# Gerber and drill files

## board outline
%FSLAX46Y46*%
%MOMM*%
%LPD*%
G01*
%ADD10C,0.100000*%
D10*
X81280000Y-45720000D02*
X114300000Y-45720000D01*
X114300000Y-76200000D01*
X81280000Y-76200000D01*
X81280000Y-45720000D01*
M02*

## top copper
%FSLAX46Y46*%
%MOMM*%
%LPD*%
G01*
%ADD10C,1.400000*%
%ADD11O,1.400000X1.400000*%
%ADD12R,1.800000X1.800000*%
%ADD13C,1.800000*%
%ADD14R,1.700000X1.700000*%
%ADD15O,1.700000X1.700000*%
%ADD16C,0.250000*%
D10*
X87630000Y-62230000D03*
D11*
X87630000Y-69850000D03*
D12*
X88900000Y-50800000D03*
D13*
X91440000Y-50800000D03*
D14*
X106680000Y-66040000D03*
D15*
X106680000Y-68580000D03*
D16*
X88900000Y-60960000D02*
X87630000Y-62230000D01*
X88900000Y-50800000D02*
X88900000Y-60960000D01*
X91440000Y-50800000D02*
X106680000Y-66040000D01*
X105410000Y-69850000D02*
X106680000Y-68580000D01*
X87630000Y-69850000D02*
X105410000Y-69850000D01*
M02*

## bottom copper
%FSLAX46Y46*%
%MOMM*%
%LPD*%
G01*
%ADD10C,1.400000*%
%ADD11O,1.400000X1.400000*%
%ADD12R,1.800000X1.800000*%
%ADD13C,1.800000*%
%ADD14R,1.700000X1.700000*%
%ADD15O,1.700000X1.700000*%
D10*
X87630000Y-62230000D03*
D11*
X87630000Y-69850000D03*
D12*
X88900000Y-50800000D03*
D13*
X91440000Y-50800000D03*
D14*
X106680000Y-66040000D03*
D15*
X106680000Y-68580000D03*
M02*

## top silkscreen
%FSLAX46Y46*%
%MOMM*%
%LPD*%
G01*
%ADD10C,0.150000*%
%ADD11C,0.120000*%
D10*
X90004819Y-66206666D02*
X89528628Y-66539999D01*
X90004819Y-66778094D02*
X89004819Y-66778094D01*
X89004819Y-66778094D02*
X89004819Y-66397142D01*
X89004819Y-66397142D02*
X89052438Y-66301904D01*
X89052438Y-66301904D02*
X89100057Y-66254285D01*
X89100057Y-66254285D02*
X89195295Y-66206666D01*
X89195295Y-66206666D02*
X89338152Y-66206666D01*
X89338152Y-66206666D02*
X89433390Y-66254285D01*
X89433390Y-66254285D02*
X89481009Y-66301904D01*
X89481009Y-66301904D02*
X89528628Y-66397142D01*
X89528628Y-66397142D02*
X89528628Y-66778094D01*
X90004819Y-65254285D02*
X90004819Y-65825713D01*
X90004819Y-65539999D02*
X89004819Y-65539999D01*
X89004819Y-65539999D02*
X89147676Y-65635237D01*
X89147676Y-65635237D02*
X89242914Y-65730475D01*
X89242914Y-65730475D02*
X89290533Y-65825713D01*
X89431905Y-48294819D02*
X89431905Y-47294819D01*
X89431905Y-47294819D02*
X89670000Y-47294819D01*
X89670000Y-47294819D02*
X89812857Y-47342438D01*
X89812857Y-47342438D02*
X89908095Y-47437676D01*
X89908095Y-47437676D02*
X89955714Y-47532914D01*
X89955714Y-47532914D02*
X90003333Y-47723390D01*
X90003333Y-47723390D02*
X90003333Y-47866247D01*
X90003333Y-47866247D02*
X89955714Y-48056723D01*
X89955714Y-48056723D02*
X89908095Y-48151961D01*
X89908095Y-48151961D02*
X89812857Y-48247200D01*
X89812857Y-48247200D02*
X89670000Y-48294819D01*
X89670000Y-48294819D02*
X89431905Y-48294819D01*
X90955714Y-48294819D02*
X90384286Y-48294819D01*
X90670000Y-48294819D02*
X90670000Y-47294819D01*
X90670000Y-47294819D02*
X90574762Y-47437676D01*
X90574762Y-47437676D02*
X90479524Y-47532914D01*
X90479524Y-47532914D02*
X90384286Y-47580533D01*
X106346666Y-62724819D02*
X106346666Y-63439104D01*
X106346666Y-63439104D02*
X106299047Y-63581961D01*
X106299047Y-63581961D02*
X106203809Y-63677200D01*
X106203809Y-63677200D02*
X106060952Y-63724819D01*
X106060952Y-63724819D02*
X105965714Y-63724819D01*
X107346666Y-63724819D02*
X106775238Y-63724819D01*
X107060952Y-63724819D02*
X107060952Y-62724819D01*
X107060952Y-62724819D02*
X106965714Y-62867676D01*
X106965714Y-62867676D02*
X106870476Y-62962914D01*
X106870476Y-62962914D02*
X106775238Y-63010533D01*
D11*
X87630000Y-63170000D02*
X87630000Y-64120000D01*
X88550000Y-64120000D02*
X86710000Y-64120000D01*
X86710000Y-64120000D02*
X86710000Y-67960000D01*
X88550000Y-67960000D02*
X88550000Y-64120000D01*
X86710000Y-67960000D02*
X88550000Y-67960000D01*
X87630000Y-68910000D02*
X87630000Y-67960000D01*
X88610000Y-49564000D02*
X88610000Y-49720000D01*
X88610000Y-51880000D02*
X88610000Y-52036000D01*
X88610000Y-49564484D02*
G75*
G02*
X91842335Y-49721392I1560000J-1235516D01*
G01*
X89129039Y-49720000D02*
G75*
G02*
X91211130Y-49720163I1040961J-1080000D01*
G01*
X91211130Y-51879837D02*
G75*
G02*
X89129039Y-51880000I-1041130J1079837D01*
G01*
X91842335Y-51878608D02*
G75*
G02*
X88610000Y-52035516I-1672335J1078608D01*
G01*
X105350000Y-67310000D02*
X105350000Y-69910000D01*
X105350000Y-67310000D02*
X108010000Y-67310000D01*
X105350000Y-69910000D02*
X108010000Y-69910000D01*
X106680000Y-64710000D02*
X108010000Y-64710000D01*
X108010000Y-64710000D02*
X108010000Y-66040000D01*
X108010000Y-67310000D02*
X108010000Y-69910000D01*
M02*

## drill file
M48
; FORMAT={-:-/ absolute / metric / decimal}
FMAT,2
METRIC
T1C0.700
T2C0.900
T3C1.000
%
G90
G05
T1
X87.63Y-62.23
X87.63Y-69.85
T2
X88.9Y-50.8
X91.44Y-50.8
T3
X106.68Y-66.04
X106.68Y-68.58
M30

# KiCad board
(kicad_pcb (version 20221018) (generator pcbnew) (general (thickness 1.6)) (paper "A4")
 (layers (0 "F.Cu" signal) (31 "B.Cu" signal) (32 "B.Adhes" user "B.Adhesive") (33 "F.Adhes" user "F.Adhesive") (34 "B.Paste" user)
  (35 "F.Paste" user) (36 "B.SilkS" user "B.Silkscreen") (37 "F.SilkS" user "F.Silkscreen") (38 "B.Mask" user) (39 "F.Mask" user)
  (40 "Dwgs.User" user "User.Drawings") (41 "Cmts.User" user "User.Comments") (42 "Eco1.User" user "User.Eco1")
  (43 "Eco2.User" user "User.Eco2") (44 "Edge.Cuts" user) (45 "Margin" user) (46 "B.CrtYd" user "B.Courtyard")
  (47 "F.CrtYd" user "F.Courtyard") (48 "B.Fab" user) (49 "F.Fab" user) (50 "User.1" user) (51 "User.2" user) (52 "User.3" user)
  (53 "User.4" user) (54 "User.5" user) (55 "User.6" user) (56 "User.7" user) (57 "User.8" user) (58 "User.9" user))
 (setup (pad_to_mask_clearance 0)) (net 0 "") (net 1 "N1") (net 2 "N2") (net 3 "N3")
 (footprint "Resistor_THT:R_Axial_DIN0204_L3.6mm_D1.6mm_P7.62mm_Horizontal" (layer "F.Cu") (at 87.63 62.23 -90)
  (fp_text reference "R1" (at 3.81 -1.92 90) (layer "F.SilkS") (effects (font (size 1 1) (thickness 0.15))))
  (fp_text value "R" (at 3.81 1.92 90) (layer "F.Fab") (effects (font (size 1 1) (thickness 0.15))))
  (fp_line (start 0.94 0) (end 1.89 0) (stroke (width 0.12) (type solid)) (layer "F.SilkS"))
  (fp_line (start 1.89 -0.92) (end 1.89 0.92) (stroke (width 0.12) (type solid)) (layer "F.SilkS"))
  (fp_line (start 1.89 0.92) (end 5.73 0.92) (stroke (width 0.12) (type solid)) (layer "F.SilkS"))
  (fp_line (start 5.73 -0.92) (end 1.89 -0.92) (stroke (width 0.12) (type solid)) (layer "F.SilkS"))
  (fp_line (start 5.73 0.92) (end 5.73 -0.92) (stroke (width 0.12) (type solid)) (layer "F.SilkS"))
  (fp_line (start 6.68 0) (end 5.73 0) (stroke (width 0.12) (type solid)) (layer "F.SilkS"))
  (pad "1" thru_hole circle (at 0 0 270) (size 1.4 1.4) (drill 0.7) (layers "*.Cu" "*.Mask") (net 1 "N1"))
  (pad "2" thru_hole oval (at 7.62 0 270) (size 1.4 1.4) (drill 0.7) (layers "*.Cu" "*.Mask") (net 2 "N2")))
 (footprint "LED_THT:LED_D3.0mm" (layer "F.Cu") (at 88.9 50.8)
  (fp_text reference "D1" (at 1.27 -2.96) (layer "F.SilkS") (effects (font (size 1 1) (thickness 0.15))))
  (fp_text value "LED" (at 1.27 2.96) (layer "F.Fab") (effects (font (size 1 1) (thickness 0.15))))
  (fp_line (start -0.29 -1.236) (end -0.29 -1.08) (stroke (width 0.12) (type solid)) (layer "F.SilkS"))
  (fp_line (start -0.29 1.08) (end -0.29 1.236) (stroke (width 0.12) (type solid)) (layer "F.SilkS"))
  (fp_arc (start -0.29 -1.235516) (mid 1.366487 -1.987659) (end 2.942335 -1.078608) (stroke (width 0.12) (type solid)) (layer "F.SilkS"))
  (fp_arc (start 0.229039 -1.08) (mid 1.270117 -1.5) (end 2.31113 -1.079837) (stroke (width 0.12) (type solid)) (layer "F.SilkS"))
  (fp_arc (start 2.31113 1.079837) (mid 1.270117 1.5) (end 0.229039 1.08) (stroke (width 0.12) (type solid)) (layer "F.SilkS"))
  (fp_arc (start 2.942335 1.078608) (mid 1.366487 1.987659) (end -0.29 1.235516) (stroke (width 0.12) (type solid)) (layer "F.SilkS"))
  (pad "1" thru_hole rect (at 0 0) (size 1.8 1.8) (drill 0.9) (layers "*.Cu" "*.Mask") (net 1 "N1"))
  (pad "2" thru_hole circle (at 2.54 0) (size 1.8 1.8) (drill 0.9) (layers "*.Cu" "*.Mask") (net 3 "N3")))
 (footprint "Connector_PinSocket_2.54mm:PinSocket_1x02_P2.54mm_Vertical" (layer "F.Cu") (at 106.68 66.04)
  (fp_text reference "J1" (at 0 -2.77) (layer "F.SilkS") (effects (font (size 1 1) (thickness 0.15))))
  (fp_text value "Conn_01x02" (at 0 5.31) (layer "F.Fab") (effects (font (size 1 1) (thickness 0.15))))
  (fp_line (start -1.33 1.27) (end -1.33 3.87) (stroke (width 0.12) (type solid)) (layer "F.SilkS"))
  (fp_line (start -1.33 1.27) (end 1.33 1.27) (stroke (width 0.12) (type solid)) (layer "F.SilkS"))
  (fp_line (start -1.33 3.87) (end 1.33 3.87) (stroke (width 0.12) (type solid)) (layer "F.SilkS"))
  (fp_line (start 0 -1.33) (end 1.33 -1.33) (stroke (width 0.12) (type solid)) (layer "F.SilkS"))
  (fp_line (start 1.33 -1.33) (end 1.33 0) (stroke (width 0.12) (type solid)) (layer "F.SilkS"))
  (fp_line (start 1.33 1.27) (end 1.33 3.87) (stroke (width 0.12) (type solid)) (layer "F.SilkS"))
  (pad "1" thru_hole rect (at 0 0) (size 1.7 1.7) (drill 1) (layers "*.Cu" "*.Mask") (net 3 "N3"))
  (pad "2" thru_hole oval (at 0 2.54) (size 1.7 1.7) (drill 1) (layers "*.Cu" "*.Mask") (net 2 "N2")))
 (gr_rect (start 81.28 45.72) (end 114.3 76.2) (stroke (width 0.1) (type default)) (fill none) (layer "Edge.Cuts"))
 (segment (start 88.9 60.96) (end 87.63 62.23) (width 0.25) (layer "F.Cu") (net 1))
 (segment (start 88.9 50.8) (end 88.9 60.96) (width 0.25) (layer "F.Cu") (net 1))
 (segment (start 91.44 50.8) (end 106.68 66.04) (width 0.25) (layer "F.Cu") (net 3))
 (segment (start 105.41 69.85) (end 106.68 68.58) (width 0.25) (layer "F.Cu") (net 2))
 (segment (start 87.63 69.85) (end 105.41 69.85) (width 0.25) (layer "F.Cu") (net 2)))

